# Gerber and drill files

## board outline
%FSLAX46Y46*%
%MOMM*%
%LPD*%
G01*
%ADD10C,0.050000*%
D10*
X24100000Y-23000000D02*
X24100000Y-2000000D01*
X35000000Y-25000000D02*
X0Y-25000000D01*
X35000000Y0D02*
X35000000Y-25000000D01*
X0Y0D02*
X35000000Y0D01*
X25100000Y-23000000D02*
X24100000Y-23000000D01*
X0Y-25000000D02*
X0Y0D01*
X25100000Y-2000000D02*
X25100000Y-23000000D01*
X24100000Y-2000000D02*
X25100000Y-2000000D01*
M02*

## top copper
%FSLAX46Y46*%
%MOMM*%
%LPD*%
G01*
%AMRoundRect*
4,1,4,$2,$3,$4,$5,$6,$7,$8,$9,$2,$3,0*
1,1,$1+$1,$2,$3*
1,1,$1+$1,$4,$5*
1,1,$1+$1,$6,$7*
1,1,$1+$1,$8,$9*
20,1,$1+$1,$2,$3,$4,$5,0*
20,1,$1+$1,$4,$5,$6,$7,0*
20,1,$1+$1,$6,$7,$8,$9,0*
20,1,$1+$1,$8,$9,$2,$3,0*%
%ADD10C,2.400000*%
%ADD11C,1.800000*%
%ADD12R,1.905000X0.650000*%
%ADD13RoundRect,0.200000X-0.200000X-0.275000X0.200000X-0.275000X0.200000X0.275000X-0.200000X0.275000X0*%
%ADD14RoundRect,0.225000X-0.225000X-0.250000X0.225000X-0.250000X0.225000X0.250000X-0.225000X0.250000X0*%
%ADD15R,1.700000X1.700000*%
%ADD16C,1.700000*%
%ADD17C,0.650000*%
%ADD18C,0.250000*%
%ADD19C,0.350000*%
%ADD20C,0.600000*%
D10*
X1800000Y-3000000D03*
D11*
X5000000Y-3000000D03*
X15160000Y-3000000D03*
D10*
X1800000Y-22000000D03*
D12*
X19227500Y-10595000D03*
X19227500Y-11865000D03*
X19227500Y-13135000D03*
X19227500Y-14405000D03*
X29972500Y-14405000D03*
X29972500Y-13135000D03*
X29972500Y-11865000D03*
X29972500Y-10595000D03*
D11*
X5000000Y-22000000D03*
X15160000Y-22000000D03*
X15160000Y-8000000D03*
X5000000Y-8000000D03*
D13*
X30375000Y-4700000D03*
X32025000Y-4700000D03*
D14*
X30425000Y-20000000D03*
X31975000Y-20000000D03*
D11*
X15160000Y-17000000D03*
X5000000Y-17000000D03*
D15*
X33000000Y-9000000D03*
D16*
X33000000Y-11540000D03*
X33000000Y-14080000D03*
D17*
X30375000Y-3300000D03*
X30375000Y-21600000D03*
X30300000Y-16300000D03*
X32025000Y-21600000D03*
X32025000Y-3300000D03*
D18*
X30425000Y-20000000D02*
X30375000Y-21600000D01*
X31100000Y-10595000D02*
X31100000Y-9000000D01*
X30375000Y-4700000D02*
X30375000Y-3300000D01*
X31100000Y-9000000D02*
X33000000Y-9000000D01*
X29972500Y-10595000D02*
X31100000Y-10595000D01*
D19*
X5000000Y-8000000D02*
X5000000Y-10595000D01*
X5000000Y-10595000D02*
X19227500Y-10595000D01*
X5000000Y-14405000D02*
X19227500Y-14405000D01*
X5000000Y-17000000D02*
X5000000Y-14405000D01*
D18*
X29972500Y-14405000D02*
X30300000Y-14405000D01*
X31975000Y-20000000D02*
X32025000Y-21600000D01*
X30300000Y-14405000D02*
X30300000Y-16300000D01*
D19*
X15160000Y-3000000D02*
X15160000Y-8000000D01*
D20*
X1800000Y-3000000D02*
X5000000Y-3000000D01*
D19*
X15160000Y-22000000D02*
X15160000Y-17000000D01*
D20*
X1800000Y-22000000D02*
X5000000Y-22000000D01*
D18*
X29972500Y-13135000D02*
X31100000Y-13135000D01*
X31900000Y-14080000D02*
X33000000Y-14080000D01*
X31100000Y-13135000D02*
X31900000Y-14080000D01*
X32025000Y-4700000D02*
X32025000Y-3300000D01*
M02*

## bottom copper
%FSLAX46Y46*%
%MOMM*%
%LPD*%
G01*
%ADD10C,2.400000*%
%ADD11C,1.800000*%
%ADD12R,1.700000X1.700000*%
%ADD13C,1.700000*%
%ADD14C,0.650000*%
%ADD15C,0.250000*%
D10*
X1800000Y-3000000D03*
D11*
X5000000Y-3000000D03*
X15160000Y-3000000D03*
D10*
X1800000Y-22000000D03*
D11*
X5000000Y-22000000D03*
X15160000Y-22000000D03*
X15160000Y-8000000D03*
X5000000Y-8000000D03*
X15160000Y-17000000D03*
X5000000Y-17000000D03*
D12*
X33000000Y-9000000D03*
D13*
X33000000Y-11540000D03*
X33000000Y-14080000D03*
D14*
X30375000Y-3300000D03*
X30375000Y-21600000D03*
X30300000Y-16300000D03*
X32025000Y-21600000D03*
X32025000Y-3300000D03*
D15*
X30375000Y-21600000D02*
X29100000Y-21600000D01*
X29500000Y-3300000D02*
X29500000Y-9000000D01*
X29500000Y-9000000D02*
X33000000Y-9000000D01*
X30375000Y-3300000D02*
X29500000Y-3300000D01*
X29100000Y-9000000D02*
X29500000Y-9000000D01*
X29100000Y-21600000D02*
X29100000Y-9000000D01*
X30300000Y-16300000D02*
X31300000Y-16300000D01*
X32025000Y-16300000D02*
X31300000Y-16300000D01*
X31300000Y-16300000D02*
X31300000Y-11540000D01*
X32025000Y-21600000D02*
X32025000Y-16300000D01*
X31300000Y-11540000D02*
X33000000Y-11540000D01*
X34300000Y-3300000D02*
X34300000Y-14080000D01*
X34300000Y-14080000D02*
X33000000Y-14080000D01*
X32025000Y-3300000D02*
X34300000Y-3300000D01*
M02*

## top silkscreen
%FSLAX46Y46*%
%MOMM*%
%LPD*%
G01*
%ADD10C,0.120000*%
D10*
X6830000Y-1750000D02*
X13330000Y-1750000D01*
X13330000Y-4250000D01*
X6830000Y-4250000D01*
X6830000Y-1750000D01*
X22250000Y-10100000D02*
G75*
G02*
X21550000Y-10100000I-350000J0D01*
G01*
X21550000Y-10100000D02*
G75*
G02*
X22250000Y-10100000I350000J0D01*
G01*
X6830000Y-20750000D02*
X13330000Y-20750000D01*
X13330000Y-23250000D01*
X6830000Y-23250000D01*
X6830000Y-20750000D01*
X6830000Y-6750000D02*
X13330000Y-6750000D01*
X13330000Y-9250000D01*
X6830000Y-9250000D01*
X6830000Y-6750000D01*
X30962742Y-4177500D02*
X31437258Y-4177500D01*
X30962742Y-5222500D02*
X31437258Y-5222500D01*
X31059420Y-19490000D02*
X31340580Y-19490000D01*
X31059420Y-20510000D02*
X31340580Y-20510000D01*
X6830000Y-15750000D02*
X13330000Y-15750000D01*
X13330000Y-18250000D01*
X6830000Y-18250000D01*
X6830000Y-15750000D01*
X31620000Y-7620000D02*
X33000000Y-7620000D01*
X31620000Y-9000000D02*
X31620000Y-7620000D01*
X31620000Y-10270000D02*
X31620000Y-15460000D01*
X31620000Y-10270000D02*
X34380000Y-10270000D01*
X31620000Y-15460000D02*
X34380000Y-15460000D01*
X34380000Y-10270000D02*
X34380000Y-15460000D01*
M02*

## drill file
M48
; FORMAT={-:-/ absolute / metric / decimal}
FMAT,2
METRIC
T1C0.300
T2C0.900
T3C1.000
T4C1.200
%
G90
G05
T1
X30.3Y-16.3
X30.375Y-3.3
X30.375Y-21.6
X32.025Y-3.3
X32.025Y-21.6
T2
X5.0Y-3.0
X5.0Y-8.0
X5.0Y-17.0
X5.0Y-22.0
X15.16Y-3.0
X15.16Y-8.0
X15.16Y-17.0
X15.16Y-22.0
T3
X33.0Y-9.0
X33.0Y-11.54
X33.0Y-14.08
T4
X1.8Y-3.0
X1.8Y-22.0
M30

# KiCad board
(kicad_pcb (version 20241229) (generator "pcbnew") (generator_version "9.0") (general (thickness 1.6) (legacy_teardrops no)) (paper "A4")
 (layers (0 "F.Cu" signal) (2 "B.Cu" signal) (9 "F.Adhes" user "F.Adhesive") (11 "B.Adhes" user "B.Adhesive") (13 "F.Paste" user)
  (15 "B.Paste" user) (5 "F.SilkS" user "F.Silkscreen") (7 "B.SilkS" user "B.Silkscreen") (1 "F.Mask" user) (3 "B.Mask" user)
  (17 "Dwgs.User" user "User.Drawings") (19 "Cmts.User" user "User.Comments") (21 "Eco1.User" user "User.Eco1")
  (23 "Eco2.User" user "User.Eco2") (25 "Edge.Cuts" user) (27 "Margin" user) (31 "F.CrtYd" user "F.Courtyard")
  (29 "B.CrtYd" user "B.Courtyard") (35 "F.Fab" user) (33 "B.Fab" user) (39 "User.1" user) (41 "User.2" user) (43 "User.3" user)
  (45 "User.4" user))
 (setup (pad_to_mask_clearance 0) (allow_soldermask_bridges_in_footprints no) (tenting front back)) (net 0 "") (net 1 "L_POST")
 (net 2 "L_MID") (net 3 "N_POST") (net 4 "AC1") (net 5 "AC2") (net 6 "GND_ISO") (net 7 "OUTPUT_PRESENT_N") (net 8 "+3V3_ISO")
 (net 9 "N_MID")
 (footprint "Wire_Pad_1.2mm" (layer "F.Cu") (at 1.8 3)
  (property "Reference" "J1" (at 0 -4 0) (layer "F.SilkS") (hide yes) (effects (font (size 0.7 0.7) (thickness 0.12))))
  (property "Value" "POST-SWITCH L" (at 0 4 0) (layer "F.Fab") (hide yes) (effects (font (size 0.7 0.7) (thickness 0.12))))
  (pad "1" thru_hole circle (at 0 0) (size 2.4 2.4) (drill 1.2) (layers "*.Cu" "*.Mask") (remove_unused_layers no) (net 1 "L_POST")))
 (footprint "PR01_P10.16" (layer "F.Cu") (at 5 3)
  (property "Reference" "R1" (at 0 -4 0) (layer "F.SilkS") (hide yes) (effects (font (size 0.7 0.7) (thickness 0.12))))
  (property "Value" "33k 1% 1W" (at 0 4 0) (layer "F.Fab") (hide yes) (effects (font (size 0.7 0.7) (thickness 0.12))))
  (fp_rect (start 1.83 -1.25) (end 8.33 1.25) (stroke (width 0.12) (type default)) (fill no) (layer "F.SilkS"))
  (pad "1" thru_hole circle (at 0 0) (size 1.8 1.8) (drill 0.9) (layers "*.Cu" "*.Mask") (remove_unused_layers no) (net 1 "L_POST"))
  (pad "2" thru_hole circle (at 10.16 0) (size 1.8 1.8) (drill 0.9) (layers "*.Cu" "*.Mask") (remove_unused_layers no) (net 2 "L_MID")))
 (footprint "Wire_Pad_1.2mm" (layer "F.Cu") (at 1.8 22)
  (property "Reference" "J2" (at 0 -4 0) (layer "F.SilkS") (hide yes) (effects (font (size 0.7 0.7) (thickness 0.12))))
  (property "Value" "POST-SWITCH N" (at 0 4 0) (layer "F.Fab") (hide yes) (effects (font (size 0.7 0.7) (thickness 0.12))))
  (pad "1" thru_hole circle (at 0 0) (size 2.4 2.4) (drill 1.2) (layers "*.Cu" "*.Mask") (remove_unused_layers no) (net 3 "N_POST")))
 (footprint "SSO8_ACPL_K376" (layer "F.Cu") (at 24.6 12.5)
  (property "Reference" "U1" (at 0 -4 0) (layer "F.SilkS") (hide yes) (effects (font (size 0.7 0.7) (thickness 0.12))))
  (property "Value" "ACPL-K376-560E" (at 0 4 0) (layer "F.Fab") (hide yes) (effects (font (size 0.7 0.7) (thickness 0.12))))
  (fp_circle (center -2.7 -2.4) (end -2.35 -2.4) (stroke (width 0.12) (type default)) (fill no) (layer "F.SilkS"))
  (pad "1" smd rect (at -5.3725 -1.905) (size 1.905 0.65) (layers "F.Cu" "F.Mask" "F.Paste") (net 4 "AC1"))
  (pad "2" smd rect (at -5.3725 -0.635) (size 1.905 0.65) (layers "F.Cu" "F.Mask" "F.Paste"))
  (pad "3" smd rect (at -5.3725 0.635) (size 1.905 0.65) (layers "F.Cu" "F.Mask" "F.Paste"))
  (pad "4" smd rect (at -5.3725 1.905) (size 1.905 0.65) (layers "F.Cu" "F.Mask" "F.Paste") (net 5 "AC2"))
  (pad "5" smd rect (at 5.3725 1.905) (size 1.905 0.65) (layers "F.Cu" "F.Mask" "F.Paste") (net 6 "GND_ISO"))
  (pad "6" smd rect (at 5.3725 0.635) (size 1.905 0.65) (layers "F.Cu" "F.Mask" "F.Paste") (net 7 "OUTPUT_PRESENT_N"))
  (pad "7" smd rect (at 5.3725 -0.635) (size 1.905 0.65) (layers "F.Cu" "F.Mask" "F.Paste"))
  (pad "8" smd rect (at 5.3725 -1.905) (size 1.905 0.65) (layers "F.Cu" "F.Mask" "F.Paste") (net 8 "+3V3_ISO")))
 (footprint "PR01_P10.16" (layer "F.Cu") (at 5 22)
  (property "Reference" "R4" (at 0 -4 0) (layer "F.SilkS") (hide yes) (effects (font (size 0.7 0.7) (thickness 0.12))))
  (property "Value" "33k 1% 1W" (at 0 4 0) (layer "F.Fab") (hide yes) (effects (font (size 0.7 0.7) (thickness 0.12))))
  (fp_rect (start 1.83 -1.25) (end 8.33 1.25) (stroke (width 0.12) (type default)) (fill no) (layer "F.SilkS"))
  (pad "1" thru_hole circle (at 0 0) (size 1.8 1.8) (drill 0.9) (layers "*.Cu" "*.Mask") (remove_unused_layers no) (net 3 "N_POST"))
  (pad "2" thru_hole circle (at 10.16 0) (size 1.8 1.8) (drill 0.9) (layers "*.Cu" "*.Mask") (remove_unused_layers no) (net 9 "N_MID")))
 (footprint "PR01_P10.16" (layer "F.Cu") (at 15.16 8 180)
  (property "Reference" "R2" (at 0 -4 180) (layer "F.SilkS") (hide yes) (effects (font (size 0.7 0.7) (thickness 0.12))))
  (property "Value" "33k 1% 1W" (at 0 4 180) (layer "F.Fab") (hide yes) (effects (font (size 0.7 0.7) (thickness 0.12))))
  (fp_rect (start 1.83 -1.25) (end 8.33 1.25) (stroke (width 0.12) (type default)) (fill no) (layer "F.SilkS"))
  (pad "1" thru_hole circle (at 0 0 180) (size 1.8 1.8) (drill 0.9) (layers "*.Cu" "*.Mask") (remove_unused_layers no) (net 2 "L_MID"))
  (pad "2" thru_hole circle (at 10.16 0 180) (size 1.8 1.8) (drill 0.9) (layers "*.Cu" "*.Mask") (remove_unused_layers no) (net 4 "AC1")))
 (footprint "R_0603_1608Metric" (layer "F.Cu") (at 31.2 4.7)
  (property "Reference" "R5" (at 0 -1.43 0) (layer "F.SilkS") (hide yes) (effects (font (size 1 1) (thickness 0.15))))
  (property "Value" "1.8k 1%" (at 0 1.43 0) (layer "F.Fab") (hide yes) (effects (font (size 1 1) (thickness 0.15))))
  (fp_line (start -0.237258 -0.5225) (end 0.237258 -0.5225) (stroke (width 0.12) (type solid)) (layer "F.SilkS"))
  (fp_line (start -0.237258 0.5225) (end 0.237258 0.5225) (stroke (width 0.12) (type solid)) (layer "F.SilkS"))
  (pad "1" smd roundrect (at -0.825 0) (size 0.8 0.95) (layers "F.Cu" "F.Mask" "F.Paste") (roundrect_rratio 0.25) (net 8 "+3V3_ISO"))
  (pad "2" smd roundrect (at 0.825 0) (size 0.8 0.95) (layers "F.Cu" "F.Mask" "F.Paste") (roundrect_rratio 0.25) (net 7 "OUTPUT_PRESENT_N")))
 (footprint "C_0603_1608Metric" (layer "F.Cu") (at 31.2 20)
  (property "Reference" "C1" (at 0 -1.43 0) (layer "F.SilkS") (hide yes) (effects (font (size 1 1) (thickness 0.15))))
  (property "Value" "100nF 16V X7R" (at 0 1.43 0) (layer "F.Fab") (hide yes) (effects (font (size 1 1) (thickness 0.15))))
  (fp_line (start -0.14058 -0.51) (end 0.14058 -0.51) (stroke (width 0.12) (type solid)) (layer "F.SilkS"))
  (fp_line (start -0.14058 0.51) (end 0.14058 0.51) (stroke (width 0.12) (type solid)) (layer "F.SilkS"))
  (pad "1" smd roundrect (at -0.775 0) (size 0.9 0.95) (layers "F.Cu" "F.Mask" "F.Paste") (roundrect_rratio 0.25) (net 8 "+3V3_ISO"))
  (pad "2" smd roundrect (at 0.775 0) (size 0.9 0.95) (layers "F.Cu" "F.Mask" "F.Paste") (roundrect_rratio 0.25) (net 6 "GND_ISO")))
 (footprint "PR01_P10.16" (layer "F.Cu") (at 15.16 17 180)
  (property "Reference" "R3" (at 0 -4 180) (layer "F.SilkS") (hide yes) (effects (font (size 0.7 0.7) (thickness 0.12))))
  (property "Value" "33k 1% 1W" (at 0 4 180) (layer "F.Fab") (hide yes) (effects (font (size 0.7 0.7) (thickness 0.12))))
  (fp_rect (start 1.83 -1.25) (end 8.33 1.25) (stroke (width 0.12) (type default)) (fill no) (layer "F.SilkS"))
  (pad "1" thru_hole circle (at 0 0 180) (size 1.8 1.8) (drill 0.9) (layers "*.Cu" "*.Mask") (remove_unused_layers no) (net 9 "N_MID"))
  (pad "2" thru_hole circle (at 10.16 0 180) (size 1.8 1.8) (drill 0.9) (layers "*.Cu" "*.Mask") (remove_unused_layers no) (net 5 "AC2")))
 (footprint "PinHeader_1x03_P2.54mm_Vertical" (layer "F.Cu") (at 33 9)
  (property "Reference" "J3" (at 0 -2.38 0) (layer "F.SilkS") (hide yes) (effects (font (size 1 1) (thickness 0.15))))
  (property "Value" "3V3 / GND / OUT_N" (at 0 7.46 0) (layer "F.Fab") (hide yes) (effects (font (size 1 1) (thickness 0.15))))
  (fp_line (start -1.38 -1.38) (end 0 -1.38) (stroke (width 0.12) (type solid)) (layer "F.SilkS"))
  (fp_line (start -1.38 0) (end -1.38 -1.38) (stroke (width 0.12) (type solid)) (layer "F.SilkS"))
  (fp_line (start -1.38 1.27) (end -1.38 6.46) (stroke (width 0.12) (type solid)) (layer "F.SilkS"))
  (fp_line (start -1.38 1.27) (end 1.38 1.27) (stroke (width 0.12) (type solid)) (layer "F.SilkS"))
  (fp_line (start -1.38 6.46) (end 1.38 6.46) (stroke (width 0.12) (type solid)) (layer "F.SilkS"))
  (fp_line (start 1.38 1.27) (end 1.38 6.46) (stroke (width 0.12) (type solid)) (layer "F.SilkS"))
  (pad "1" thru_hole rect (at 0 0) (size 1.7 1.7) (drill 1) (layers "*.Cu" "*.Mask") (remove_unused_layers no) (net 8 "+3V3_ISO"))
  (pad "2" thru_hole circle (at 0 2.54) (size 1.7 1.7) (drill 1) (layers "*.Cu" "*.Mask") (remove_unused_layers no) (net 6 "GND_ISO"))
  (pad "3" thru_hole circle (at 0 5.08) (size 1.7 1.7) (drill 1) (layers "*.Cu" "*.Mask") (remove_unused_layers no)
   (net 7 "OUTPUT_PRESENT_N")))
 (gr_line (start 24.1 23) (end 24.1 2) (stroke (width 0.05) (type default)) (layer "Edge.Cuts"))
 (gr_line (start 35 25) (end 0 25) (stroke (width 0.05) (type default)) (layer "Edge.Cuts"))
 (gr_line (start 35 0) (end 35 25) (stroke (width 0.05) (type default)) (layer "Edge.Cuts"))
 (gr_line (start 0 0) (end 35 0) (stroke (width 0.05) (type default)) (layer "Edge.Cuts"))
 (gr_line (start 25.1 23) (end 24.1 23) (stroke (width 0.05) (type default)) (layer "Edge.Cuts"))
 (gr_line (start 0 25) (end 0 0) (stroke (width 0.05) (type default)) (layer "Edge.Cuts"))
 (gr_line (start 25.1 2) (end 25.1 23) (stroke (width 0.05) (type default)) (layer "Edge.Cuts"))
 (gr_line (start 24.1 2) (end 25.1 2) (stroke (width 0.05) (type default)) (layer "Edge.Cuts"))
 (segment (start 30.425 20) (end 30.375 21.6) (width 0.25) (layer "F.Cu") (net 8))
 (segment (start 31.1 10.595) (end 31.1 9) (width 0.25) (layer "F.Cu") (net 8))
 (segment (start 30.375 4.7) (end 30.375 3.3) (width 0.25) (layer "F.Cu") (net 8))
 (segment (start 31.1 9) (end 33 9) (width 0.25) (layer "F.Cu") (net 8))
 (segment (start 29.9725 10.595) (end 31.1 10.595) (width 0.25) (layer "F.Cu") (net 8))
 (via (at 30.375 3.3) (size 0.65) (drill 0.3) (layers "F.Cu" "B.Cu") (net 8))
 (via (at 30.375 21.6) (size 0.65) (drill 0.3) (layers "F.Cu" "B.Cu") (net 8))
 (segment (start 30.375 21.6) (end 29.1 21.6) (width 0.25) (layer "B.Cu") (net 8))
 (segment (start 29.5 3.3) (end 29.5 9) (width 0.25) (layer "B.Cu") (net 8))
 (segment (start 29.5 9) (end 33 9) (width 0.25) (layer "B.Cu") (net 8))
 (segment (start 30.375 3.3) (end 29.5 3.3) (width 0.25) (layer "B.Cu") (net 8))
 (segment (start 29.1 9) (end 29.5 9) (width 0.25) (layer "B.Cu") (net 8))
 (segment (start 29.1 21.6) (end 29.1 9) (width 0.25) (layer "B.Cu") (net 8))
 (segment (start 5 8) (end 5 10.595) (width 0.35) (layer "F.Cu") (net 4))
 (segment (start 5 10.595) (end 19.2275 10.595) (width 0.35) (layer "F.Cu") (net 4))
 (segment (start 5 14.405) (end 19.2275 14.405) (width 0.35) (layer "F.Cu") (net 5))
 (segment (start 5 17) (end 5 14.405) (width 0.35) (layer "F.Cu") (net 5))
 (segment (start 29.9725 14.405) (end 30.3 14.405) (width 0.25) (layer "F.Cu") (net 6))
 (segment (start 31.975 20) (end 32.025 21.6) (width 0.25) (layer "F.Cu") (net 6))
 (segment (start 30.3 14.405) (end 30.3 16.3) (width 0.25) (layer "F.Cu") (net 6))
 (via (at 30.3 16.3) (size 0.65) (drill 0.3) (layers "F.Cu" "B.Cu") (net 6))
 (via (at 32.025 21.6) (size 0.65) (drill 0.3) (layers "F.Cu" "B.Cu") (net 6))
 (segment (start 30.3 16.3) (end 31.3 16.3) (width 0.25) (layer "B.Cu") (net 6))
 (segment (start 32.025 16.3) (end 31.3 16.3) (width 0.25) (layer "B.Cu") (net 6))
 (segment (start 31.3 16.3) (end 31.3 11.54) (width 0.25) (layer "B.Cu") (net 6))
 (segment (start 32.025 21.6) (end 32.025 16.3) (width 0.25) (layer "B.Cu") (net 6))
 (segment (start 31.3 11.54) (end 33 11.54) (width 0.25) (layer "B.Cu") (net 6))
 (segment (start 15.16 3) (end 15.16 8) (width 0.35) (layer "F.Cu") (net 2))
 (segment (start 1.8 3) (end 5 3) (width 0.6) (layer "F.Cu") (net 1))
 (segment (start 15.16 22) (end 15.16 17) (width 0.35) (layer "F.Cu") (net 9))
 (segment (start 1.8 22) (end 5 22) (width 0.6) (layer "F.Cu") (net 3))
 (segment (start 29.9725 13.135) (end 31.1 13.135) (width 0.25) (layer "F.Cu") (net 7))
 (segment (start 31.9 14.08) (end 33 14.08) (width 0.25) (layer "F.Cu") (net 7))
 (segment (start 31.1 13.135) (end 31.9 14.08) (width 0.25) (layer "F.Cu") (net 7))
 (segment (start 32.025 4.7) (end 32.025 3.3) (width 0.25) (layer "F.Cu") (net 7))
 (via (at 32.025 3.3) (size 0.65) (drill 0.3) (layers "F.Cu" "B.Cu") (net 7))
 (segment (start 34.3 3.3) (end 34.3 14.08) (width 0.25) (layer "B.Cu") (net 7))
 (segment (start 34.3 14.08) (end 33 14.08) (width 0.25) (layer "B.Cu") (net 7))
 (segment (start 32.025 3.3) (end 34.3 3.3) (width 0.25) (layer "B.Cu") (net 7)))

